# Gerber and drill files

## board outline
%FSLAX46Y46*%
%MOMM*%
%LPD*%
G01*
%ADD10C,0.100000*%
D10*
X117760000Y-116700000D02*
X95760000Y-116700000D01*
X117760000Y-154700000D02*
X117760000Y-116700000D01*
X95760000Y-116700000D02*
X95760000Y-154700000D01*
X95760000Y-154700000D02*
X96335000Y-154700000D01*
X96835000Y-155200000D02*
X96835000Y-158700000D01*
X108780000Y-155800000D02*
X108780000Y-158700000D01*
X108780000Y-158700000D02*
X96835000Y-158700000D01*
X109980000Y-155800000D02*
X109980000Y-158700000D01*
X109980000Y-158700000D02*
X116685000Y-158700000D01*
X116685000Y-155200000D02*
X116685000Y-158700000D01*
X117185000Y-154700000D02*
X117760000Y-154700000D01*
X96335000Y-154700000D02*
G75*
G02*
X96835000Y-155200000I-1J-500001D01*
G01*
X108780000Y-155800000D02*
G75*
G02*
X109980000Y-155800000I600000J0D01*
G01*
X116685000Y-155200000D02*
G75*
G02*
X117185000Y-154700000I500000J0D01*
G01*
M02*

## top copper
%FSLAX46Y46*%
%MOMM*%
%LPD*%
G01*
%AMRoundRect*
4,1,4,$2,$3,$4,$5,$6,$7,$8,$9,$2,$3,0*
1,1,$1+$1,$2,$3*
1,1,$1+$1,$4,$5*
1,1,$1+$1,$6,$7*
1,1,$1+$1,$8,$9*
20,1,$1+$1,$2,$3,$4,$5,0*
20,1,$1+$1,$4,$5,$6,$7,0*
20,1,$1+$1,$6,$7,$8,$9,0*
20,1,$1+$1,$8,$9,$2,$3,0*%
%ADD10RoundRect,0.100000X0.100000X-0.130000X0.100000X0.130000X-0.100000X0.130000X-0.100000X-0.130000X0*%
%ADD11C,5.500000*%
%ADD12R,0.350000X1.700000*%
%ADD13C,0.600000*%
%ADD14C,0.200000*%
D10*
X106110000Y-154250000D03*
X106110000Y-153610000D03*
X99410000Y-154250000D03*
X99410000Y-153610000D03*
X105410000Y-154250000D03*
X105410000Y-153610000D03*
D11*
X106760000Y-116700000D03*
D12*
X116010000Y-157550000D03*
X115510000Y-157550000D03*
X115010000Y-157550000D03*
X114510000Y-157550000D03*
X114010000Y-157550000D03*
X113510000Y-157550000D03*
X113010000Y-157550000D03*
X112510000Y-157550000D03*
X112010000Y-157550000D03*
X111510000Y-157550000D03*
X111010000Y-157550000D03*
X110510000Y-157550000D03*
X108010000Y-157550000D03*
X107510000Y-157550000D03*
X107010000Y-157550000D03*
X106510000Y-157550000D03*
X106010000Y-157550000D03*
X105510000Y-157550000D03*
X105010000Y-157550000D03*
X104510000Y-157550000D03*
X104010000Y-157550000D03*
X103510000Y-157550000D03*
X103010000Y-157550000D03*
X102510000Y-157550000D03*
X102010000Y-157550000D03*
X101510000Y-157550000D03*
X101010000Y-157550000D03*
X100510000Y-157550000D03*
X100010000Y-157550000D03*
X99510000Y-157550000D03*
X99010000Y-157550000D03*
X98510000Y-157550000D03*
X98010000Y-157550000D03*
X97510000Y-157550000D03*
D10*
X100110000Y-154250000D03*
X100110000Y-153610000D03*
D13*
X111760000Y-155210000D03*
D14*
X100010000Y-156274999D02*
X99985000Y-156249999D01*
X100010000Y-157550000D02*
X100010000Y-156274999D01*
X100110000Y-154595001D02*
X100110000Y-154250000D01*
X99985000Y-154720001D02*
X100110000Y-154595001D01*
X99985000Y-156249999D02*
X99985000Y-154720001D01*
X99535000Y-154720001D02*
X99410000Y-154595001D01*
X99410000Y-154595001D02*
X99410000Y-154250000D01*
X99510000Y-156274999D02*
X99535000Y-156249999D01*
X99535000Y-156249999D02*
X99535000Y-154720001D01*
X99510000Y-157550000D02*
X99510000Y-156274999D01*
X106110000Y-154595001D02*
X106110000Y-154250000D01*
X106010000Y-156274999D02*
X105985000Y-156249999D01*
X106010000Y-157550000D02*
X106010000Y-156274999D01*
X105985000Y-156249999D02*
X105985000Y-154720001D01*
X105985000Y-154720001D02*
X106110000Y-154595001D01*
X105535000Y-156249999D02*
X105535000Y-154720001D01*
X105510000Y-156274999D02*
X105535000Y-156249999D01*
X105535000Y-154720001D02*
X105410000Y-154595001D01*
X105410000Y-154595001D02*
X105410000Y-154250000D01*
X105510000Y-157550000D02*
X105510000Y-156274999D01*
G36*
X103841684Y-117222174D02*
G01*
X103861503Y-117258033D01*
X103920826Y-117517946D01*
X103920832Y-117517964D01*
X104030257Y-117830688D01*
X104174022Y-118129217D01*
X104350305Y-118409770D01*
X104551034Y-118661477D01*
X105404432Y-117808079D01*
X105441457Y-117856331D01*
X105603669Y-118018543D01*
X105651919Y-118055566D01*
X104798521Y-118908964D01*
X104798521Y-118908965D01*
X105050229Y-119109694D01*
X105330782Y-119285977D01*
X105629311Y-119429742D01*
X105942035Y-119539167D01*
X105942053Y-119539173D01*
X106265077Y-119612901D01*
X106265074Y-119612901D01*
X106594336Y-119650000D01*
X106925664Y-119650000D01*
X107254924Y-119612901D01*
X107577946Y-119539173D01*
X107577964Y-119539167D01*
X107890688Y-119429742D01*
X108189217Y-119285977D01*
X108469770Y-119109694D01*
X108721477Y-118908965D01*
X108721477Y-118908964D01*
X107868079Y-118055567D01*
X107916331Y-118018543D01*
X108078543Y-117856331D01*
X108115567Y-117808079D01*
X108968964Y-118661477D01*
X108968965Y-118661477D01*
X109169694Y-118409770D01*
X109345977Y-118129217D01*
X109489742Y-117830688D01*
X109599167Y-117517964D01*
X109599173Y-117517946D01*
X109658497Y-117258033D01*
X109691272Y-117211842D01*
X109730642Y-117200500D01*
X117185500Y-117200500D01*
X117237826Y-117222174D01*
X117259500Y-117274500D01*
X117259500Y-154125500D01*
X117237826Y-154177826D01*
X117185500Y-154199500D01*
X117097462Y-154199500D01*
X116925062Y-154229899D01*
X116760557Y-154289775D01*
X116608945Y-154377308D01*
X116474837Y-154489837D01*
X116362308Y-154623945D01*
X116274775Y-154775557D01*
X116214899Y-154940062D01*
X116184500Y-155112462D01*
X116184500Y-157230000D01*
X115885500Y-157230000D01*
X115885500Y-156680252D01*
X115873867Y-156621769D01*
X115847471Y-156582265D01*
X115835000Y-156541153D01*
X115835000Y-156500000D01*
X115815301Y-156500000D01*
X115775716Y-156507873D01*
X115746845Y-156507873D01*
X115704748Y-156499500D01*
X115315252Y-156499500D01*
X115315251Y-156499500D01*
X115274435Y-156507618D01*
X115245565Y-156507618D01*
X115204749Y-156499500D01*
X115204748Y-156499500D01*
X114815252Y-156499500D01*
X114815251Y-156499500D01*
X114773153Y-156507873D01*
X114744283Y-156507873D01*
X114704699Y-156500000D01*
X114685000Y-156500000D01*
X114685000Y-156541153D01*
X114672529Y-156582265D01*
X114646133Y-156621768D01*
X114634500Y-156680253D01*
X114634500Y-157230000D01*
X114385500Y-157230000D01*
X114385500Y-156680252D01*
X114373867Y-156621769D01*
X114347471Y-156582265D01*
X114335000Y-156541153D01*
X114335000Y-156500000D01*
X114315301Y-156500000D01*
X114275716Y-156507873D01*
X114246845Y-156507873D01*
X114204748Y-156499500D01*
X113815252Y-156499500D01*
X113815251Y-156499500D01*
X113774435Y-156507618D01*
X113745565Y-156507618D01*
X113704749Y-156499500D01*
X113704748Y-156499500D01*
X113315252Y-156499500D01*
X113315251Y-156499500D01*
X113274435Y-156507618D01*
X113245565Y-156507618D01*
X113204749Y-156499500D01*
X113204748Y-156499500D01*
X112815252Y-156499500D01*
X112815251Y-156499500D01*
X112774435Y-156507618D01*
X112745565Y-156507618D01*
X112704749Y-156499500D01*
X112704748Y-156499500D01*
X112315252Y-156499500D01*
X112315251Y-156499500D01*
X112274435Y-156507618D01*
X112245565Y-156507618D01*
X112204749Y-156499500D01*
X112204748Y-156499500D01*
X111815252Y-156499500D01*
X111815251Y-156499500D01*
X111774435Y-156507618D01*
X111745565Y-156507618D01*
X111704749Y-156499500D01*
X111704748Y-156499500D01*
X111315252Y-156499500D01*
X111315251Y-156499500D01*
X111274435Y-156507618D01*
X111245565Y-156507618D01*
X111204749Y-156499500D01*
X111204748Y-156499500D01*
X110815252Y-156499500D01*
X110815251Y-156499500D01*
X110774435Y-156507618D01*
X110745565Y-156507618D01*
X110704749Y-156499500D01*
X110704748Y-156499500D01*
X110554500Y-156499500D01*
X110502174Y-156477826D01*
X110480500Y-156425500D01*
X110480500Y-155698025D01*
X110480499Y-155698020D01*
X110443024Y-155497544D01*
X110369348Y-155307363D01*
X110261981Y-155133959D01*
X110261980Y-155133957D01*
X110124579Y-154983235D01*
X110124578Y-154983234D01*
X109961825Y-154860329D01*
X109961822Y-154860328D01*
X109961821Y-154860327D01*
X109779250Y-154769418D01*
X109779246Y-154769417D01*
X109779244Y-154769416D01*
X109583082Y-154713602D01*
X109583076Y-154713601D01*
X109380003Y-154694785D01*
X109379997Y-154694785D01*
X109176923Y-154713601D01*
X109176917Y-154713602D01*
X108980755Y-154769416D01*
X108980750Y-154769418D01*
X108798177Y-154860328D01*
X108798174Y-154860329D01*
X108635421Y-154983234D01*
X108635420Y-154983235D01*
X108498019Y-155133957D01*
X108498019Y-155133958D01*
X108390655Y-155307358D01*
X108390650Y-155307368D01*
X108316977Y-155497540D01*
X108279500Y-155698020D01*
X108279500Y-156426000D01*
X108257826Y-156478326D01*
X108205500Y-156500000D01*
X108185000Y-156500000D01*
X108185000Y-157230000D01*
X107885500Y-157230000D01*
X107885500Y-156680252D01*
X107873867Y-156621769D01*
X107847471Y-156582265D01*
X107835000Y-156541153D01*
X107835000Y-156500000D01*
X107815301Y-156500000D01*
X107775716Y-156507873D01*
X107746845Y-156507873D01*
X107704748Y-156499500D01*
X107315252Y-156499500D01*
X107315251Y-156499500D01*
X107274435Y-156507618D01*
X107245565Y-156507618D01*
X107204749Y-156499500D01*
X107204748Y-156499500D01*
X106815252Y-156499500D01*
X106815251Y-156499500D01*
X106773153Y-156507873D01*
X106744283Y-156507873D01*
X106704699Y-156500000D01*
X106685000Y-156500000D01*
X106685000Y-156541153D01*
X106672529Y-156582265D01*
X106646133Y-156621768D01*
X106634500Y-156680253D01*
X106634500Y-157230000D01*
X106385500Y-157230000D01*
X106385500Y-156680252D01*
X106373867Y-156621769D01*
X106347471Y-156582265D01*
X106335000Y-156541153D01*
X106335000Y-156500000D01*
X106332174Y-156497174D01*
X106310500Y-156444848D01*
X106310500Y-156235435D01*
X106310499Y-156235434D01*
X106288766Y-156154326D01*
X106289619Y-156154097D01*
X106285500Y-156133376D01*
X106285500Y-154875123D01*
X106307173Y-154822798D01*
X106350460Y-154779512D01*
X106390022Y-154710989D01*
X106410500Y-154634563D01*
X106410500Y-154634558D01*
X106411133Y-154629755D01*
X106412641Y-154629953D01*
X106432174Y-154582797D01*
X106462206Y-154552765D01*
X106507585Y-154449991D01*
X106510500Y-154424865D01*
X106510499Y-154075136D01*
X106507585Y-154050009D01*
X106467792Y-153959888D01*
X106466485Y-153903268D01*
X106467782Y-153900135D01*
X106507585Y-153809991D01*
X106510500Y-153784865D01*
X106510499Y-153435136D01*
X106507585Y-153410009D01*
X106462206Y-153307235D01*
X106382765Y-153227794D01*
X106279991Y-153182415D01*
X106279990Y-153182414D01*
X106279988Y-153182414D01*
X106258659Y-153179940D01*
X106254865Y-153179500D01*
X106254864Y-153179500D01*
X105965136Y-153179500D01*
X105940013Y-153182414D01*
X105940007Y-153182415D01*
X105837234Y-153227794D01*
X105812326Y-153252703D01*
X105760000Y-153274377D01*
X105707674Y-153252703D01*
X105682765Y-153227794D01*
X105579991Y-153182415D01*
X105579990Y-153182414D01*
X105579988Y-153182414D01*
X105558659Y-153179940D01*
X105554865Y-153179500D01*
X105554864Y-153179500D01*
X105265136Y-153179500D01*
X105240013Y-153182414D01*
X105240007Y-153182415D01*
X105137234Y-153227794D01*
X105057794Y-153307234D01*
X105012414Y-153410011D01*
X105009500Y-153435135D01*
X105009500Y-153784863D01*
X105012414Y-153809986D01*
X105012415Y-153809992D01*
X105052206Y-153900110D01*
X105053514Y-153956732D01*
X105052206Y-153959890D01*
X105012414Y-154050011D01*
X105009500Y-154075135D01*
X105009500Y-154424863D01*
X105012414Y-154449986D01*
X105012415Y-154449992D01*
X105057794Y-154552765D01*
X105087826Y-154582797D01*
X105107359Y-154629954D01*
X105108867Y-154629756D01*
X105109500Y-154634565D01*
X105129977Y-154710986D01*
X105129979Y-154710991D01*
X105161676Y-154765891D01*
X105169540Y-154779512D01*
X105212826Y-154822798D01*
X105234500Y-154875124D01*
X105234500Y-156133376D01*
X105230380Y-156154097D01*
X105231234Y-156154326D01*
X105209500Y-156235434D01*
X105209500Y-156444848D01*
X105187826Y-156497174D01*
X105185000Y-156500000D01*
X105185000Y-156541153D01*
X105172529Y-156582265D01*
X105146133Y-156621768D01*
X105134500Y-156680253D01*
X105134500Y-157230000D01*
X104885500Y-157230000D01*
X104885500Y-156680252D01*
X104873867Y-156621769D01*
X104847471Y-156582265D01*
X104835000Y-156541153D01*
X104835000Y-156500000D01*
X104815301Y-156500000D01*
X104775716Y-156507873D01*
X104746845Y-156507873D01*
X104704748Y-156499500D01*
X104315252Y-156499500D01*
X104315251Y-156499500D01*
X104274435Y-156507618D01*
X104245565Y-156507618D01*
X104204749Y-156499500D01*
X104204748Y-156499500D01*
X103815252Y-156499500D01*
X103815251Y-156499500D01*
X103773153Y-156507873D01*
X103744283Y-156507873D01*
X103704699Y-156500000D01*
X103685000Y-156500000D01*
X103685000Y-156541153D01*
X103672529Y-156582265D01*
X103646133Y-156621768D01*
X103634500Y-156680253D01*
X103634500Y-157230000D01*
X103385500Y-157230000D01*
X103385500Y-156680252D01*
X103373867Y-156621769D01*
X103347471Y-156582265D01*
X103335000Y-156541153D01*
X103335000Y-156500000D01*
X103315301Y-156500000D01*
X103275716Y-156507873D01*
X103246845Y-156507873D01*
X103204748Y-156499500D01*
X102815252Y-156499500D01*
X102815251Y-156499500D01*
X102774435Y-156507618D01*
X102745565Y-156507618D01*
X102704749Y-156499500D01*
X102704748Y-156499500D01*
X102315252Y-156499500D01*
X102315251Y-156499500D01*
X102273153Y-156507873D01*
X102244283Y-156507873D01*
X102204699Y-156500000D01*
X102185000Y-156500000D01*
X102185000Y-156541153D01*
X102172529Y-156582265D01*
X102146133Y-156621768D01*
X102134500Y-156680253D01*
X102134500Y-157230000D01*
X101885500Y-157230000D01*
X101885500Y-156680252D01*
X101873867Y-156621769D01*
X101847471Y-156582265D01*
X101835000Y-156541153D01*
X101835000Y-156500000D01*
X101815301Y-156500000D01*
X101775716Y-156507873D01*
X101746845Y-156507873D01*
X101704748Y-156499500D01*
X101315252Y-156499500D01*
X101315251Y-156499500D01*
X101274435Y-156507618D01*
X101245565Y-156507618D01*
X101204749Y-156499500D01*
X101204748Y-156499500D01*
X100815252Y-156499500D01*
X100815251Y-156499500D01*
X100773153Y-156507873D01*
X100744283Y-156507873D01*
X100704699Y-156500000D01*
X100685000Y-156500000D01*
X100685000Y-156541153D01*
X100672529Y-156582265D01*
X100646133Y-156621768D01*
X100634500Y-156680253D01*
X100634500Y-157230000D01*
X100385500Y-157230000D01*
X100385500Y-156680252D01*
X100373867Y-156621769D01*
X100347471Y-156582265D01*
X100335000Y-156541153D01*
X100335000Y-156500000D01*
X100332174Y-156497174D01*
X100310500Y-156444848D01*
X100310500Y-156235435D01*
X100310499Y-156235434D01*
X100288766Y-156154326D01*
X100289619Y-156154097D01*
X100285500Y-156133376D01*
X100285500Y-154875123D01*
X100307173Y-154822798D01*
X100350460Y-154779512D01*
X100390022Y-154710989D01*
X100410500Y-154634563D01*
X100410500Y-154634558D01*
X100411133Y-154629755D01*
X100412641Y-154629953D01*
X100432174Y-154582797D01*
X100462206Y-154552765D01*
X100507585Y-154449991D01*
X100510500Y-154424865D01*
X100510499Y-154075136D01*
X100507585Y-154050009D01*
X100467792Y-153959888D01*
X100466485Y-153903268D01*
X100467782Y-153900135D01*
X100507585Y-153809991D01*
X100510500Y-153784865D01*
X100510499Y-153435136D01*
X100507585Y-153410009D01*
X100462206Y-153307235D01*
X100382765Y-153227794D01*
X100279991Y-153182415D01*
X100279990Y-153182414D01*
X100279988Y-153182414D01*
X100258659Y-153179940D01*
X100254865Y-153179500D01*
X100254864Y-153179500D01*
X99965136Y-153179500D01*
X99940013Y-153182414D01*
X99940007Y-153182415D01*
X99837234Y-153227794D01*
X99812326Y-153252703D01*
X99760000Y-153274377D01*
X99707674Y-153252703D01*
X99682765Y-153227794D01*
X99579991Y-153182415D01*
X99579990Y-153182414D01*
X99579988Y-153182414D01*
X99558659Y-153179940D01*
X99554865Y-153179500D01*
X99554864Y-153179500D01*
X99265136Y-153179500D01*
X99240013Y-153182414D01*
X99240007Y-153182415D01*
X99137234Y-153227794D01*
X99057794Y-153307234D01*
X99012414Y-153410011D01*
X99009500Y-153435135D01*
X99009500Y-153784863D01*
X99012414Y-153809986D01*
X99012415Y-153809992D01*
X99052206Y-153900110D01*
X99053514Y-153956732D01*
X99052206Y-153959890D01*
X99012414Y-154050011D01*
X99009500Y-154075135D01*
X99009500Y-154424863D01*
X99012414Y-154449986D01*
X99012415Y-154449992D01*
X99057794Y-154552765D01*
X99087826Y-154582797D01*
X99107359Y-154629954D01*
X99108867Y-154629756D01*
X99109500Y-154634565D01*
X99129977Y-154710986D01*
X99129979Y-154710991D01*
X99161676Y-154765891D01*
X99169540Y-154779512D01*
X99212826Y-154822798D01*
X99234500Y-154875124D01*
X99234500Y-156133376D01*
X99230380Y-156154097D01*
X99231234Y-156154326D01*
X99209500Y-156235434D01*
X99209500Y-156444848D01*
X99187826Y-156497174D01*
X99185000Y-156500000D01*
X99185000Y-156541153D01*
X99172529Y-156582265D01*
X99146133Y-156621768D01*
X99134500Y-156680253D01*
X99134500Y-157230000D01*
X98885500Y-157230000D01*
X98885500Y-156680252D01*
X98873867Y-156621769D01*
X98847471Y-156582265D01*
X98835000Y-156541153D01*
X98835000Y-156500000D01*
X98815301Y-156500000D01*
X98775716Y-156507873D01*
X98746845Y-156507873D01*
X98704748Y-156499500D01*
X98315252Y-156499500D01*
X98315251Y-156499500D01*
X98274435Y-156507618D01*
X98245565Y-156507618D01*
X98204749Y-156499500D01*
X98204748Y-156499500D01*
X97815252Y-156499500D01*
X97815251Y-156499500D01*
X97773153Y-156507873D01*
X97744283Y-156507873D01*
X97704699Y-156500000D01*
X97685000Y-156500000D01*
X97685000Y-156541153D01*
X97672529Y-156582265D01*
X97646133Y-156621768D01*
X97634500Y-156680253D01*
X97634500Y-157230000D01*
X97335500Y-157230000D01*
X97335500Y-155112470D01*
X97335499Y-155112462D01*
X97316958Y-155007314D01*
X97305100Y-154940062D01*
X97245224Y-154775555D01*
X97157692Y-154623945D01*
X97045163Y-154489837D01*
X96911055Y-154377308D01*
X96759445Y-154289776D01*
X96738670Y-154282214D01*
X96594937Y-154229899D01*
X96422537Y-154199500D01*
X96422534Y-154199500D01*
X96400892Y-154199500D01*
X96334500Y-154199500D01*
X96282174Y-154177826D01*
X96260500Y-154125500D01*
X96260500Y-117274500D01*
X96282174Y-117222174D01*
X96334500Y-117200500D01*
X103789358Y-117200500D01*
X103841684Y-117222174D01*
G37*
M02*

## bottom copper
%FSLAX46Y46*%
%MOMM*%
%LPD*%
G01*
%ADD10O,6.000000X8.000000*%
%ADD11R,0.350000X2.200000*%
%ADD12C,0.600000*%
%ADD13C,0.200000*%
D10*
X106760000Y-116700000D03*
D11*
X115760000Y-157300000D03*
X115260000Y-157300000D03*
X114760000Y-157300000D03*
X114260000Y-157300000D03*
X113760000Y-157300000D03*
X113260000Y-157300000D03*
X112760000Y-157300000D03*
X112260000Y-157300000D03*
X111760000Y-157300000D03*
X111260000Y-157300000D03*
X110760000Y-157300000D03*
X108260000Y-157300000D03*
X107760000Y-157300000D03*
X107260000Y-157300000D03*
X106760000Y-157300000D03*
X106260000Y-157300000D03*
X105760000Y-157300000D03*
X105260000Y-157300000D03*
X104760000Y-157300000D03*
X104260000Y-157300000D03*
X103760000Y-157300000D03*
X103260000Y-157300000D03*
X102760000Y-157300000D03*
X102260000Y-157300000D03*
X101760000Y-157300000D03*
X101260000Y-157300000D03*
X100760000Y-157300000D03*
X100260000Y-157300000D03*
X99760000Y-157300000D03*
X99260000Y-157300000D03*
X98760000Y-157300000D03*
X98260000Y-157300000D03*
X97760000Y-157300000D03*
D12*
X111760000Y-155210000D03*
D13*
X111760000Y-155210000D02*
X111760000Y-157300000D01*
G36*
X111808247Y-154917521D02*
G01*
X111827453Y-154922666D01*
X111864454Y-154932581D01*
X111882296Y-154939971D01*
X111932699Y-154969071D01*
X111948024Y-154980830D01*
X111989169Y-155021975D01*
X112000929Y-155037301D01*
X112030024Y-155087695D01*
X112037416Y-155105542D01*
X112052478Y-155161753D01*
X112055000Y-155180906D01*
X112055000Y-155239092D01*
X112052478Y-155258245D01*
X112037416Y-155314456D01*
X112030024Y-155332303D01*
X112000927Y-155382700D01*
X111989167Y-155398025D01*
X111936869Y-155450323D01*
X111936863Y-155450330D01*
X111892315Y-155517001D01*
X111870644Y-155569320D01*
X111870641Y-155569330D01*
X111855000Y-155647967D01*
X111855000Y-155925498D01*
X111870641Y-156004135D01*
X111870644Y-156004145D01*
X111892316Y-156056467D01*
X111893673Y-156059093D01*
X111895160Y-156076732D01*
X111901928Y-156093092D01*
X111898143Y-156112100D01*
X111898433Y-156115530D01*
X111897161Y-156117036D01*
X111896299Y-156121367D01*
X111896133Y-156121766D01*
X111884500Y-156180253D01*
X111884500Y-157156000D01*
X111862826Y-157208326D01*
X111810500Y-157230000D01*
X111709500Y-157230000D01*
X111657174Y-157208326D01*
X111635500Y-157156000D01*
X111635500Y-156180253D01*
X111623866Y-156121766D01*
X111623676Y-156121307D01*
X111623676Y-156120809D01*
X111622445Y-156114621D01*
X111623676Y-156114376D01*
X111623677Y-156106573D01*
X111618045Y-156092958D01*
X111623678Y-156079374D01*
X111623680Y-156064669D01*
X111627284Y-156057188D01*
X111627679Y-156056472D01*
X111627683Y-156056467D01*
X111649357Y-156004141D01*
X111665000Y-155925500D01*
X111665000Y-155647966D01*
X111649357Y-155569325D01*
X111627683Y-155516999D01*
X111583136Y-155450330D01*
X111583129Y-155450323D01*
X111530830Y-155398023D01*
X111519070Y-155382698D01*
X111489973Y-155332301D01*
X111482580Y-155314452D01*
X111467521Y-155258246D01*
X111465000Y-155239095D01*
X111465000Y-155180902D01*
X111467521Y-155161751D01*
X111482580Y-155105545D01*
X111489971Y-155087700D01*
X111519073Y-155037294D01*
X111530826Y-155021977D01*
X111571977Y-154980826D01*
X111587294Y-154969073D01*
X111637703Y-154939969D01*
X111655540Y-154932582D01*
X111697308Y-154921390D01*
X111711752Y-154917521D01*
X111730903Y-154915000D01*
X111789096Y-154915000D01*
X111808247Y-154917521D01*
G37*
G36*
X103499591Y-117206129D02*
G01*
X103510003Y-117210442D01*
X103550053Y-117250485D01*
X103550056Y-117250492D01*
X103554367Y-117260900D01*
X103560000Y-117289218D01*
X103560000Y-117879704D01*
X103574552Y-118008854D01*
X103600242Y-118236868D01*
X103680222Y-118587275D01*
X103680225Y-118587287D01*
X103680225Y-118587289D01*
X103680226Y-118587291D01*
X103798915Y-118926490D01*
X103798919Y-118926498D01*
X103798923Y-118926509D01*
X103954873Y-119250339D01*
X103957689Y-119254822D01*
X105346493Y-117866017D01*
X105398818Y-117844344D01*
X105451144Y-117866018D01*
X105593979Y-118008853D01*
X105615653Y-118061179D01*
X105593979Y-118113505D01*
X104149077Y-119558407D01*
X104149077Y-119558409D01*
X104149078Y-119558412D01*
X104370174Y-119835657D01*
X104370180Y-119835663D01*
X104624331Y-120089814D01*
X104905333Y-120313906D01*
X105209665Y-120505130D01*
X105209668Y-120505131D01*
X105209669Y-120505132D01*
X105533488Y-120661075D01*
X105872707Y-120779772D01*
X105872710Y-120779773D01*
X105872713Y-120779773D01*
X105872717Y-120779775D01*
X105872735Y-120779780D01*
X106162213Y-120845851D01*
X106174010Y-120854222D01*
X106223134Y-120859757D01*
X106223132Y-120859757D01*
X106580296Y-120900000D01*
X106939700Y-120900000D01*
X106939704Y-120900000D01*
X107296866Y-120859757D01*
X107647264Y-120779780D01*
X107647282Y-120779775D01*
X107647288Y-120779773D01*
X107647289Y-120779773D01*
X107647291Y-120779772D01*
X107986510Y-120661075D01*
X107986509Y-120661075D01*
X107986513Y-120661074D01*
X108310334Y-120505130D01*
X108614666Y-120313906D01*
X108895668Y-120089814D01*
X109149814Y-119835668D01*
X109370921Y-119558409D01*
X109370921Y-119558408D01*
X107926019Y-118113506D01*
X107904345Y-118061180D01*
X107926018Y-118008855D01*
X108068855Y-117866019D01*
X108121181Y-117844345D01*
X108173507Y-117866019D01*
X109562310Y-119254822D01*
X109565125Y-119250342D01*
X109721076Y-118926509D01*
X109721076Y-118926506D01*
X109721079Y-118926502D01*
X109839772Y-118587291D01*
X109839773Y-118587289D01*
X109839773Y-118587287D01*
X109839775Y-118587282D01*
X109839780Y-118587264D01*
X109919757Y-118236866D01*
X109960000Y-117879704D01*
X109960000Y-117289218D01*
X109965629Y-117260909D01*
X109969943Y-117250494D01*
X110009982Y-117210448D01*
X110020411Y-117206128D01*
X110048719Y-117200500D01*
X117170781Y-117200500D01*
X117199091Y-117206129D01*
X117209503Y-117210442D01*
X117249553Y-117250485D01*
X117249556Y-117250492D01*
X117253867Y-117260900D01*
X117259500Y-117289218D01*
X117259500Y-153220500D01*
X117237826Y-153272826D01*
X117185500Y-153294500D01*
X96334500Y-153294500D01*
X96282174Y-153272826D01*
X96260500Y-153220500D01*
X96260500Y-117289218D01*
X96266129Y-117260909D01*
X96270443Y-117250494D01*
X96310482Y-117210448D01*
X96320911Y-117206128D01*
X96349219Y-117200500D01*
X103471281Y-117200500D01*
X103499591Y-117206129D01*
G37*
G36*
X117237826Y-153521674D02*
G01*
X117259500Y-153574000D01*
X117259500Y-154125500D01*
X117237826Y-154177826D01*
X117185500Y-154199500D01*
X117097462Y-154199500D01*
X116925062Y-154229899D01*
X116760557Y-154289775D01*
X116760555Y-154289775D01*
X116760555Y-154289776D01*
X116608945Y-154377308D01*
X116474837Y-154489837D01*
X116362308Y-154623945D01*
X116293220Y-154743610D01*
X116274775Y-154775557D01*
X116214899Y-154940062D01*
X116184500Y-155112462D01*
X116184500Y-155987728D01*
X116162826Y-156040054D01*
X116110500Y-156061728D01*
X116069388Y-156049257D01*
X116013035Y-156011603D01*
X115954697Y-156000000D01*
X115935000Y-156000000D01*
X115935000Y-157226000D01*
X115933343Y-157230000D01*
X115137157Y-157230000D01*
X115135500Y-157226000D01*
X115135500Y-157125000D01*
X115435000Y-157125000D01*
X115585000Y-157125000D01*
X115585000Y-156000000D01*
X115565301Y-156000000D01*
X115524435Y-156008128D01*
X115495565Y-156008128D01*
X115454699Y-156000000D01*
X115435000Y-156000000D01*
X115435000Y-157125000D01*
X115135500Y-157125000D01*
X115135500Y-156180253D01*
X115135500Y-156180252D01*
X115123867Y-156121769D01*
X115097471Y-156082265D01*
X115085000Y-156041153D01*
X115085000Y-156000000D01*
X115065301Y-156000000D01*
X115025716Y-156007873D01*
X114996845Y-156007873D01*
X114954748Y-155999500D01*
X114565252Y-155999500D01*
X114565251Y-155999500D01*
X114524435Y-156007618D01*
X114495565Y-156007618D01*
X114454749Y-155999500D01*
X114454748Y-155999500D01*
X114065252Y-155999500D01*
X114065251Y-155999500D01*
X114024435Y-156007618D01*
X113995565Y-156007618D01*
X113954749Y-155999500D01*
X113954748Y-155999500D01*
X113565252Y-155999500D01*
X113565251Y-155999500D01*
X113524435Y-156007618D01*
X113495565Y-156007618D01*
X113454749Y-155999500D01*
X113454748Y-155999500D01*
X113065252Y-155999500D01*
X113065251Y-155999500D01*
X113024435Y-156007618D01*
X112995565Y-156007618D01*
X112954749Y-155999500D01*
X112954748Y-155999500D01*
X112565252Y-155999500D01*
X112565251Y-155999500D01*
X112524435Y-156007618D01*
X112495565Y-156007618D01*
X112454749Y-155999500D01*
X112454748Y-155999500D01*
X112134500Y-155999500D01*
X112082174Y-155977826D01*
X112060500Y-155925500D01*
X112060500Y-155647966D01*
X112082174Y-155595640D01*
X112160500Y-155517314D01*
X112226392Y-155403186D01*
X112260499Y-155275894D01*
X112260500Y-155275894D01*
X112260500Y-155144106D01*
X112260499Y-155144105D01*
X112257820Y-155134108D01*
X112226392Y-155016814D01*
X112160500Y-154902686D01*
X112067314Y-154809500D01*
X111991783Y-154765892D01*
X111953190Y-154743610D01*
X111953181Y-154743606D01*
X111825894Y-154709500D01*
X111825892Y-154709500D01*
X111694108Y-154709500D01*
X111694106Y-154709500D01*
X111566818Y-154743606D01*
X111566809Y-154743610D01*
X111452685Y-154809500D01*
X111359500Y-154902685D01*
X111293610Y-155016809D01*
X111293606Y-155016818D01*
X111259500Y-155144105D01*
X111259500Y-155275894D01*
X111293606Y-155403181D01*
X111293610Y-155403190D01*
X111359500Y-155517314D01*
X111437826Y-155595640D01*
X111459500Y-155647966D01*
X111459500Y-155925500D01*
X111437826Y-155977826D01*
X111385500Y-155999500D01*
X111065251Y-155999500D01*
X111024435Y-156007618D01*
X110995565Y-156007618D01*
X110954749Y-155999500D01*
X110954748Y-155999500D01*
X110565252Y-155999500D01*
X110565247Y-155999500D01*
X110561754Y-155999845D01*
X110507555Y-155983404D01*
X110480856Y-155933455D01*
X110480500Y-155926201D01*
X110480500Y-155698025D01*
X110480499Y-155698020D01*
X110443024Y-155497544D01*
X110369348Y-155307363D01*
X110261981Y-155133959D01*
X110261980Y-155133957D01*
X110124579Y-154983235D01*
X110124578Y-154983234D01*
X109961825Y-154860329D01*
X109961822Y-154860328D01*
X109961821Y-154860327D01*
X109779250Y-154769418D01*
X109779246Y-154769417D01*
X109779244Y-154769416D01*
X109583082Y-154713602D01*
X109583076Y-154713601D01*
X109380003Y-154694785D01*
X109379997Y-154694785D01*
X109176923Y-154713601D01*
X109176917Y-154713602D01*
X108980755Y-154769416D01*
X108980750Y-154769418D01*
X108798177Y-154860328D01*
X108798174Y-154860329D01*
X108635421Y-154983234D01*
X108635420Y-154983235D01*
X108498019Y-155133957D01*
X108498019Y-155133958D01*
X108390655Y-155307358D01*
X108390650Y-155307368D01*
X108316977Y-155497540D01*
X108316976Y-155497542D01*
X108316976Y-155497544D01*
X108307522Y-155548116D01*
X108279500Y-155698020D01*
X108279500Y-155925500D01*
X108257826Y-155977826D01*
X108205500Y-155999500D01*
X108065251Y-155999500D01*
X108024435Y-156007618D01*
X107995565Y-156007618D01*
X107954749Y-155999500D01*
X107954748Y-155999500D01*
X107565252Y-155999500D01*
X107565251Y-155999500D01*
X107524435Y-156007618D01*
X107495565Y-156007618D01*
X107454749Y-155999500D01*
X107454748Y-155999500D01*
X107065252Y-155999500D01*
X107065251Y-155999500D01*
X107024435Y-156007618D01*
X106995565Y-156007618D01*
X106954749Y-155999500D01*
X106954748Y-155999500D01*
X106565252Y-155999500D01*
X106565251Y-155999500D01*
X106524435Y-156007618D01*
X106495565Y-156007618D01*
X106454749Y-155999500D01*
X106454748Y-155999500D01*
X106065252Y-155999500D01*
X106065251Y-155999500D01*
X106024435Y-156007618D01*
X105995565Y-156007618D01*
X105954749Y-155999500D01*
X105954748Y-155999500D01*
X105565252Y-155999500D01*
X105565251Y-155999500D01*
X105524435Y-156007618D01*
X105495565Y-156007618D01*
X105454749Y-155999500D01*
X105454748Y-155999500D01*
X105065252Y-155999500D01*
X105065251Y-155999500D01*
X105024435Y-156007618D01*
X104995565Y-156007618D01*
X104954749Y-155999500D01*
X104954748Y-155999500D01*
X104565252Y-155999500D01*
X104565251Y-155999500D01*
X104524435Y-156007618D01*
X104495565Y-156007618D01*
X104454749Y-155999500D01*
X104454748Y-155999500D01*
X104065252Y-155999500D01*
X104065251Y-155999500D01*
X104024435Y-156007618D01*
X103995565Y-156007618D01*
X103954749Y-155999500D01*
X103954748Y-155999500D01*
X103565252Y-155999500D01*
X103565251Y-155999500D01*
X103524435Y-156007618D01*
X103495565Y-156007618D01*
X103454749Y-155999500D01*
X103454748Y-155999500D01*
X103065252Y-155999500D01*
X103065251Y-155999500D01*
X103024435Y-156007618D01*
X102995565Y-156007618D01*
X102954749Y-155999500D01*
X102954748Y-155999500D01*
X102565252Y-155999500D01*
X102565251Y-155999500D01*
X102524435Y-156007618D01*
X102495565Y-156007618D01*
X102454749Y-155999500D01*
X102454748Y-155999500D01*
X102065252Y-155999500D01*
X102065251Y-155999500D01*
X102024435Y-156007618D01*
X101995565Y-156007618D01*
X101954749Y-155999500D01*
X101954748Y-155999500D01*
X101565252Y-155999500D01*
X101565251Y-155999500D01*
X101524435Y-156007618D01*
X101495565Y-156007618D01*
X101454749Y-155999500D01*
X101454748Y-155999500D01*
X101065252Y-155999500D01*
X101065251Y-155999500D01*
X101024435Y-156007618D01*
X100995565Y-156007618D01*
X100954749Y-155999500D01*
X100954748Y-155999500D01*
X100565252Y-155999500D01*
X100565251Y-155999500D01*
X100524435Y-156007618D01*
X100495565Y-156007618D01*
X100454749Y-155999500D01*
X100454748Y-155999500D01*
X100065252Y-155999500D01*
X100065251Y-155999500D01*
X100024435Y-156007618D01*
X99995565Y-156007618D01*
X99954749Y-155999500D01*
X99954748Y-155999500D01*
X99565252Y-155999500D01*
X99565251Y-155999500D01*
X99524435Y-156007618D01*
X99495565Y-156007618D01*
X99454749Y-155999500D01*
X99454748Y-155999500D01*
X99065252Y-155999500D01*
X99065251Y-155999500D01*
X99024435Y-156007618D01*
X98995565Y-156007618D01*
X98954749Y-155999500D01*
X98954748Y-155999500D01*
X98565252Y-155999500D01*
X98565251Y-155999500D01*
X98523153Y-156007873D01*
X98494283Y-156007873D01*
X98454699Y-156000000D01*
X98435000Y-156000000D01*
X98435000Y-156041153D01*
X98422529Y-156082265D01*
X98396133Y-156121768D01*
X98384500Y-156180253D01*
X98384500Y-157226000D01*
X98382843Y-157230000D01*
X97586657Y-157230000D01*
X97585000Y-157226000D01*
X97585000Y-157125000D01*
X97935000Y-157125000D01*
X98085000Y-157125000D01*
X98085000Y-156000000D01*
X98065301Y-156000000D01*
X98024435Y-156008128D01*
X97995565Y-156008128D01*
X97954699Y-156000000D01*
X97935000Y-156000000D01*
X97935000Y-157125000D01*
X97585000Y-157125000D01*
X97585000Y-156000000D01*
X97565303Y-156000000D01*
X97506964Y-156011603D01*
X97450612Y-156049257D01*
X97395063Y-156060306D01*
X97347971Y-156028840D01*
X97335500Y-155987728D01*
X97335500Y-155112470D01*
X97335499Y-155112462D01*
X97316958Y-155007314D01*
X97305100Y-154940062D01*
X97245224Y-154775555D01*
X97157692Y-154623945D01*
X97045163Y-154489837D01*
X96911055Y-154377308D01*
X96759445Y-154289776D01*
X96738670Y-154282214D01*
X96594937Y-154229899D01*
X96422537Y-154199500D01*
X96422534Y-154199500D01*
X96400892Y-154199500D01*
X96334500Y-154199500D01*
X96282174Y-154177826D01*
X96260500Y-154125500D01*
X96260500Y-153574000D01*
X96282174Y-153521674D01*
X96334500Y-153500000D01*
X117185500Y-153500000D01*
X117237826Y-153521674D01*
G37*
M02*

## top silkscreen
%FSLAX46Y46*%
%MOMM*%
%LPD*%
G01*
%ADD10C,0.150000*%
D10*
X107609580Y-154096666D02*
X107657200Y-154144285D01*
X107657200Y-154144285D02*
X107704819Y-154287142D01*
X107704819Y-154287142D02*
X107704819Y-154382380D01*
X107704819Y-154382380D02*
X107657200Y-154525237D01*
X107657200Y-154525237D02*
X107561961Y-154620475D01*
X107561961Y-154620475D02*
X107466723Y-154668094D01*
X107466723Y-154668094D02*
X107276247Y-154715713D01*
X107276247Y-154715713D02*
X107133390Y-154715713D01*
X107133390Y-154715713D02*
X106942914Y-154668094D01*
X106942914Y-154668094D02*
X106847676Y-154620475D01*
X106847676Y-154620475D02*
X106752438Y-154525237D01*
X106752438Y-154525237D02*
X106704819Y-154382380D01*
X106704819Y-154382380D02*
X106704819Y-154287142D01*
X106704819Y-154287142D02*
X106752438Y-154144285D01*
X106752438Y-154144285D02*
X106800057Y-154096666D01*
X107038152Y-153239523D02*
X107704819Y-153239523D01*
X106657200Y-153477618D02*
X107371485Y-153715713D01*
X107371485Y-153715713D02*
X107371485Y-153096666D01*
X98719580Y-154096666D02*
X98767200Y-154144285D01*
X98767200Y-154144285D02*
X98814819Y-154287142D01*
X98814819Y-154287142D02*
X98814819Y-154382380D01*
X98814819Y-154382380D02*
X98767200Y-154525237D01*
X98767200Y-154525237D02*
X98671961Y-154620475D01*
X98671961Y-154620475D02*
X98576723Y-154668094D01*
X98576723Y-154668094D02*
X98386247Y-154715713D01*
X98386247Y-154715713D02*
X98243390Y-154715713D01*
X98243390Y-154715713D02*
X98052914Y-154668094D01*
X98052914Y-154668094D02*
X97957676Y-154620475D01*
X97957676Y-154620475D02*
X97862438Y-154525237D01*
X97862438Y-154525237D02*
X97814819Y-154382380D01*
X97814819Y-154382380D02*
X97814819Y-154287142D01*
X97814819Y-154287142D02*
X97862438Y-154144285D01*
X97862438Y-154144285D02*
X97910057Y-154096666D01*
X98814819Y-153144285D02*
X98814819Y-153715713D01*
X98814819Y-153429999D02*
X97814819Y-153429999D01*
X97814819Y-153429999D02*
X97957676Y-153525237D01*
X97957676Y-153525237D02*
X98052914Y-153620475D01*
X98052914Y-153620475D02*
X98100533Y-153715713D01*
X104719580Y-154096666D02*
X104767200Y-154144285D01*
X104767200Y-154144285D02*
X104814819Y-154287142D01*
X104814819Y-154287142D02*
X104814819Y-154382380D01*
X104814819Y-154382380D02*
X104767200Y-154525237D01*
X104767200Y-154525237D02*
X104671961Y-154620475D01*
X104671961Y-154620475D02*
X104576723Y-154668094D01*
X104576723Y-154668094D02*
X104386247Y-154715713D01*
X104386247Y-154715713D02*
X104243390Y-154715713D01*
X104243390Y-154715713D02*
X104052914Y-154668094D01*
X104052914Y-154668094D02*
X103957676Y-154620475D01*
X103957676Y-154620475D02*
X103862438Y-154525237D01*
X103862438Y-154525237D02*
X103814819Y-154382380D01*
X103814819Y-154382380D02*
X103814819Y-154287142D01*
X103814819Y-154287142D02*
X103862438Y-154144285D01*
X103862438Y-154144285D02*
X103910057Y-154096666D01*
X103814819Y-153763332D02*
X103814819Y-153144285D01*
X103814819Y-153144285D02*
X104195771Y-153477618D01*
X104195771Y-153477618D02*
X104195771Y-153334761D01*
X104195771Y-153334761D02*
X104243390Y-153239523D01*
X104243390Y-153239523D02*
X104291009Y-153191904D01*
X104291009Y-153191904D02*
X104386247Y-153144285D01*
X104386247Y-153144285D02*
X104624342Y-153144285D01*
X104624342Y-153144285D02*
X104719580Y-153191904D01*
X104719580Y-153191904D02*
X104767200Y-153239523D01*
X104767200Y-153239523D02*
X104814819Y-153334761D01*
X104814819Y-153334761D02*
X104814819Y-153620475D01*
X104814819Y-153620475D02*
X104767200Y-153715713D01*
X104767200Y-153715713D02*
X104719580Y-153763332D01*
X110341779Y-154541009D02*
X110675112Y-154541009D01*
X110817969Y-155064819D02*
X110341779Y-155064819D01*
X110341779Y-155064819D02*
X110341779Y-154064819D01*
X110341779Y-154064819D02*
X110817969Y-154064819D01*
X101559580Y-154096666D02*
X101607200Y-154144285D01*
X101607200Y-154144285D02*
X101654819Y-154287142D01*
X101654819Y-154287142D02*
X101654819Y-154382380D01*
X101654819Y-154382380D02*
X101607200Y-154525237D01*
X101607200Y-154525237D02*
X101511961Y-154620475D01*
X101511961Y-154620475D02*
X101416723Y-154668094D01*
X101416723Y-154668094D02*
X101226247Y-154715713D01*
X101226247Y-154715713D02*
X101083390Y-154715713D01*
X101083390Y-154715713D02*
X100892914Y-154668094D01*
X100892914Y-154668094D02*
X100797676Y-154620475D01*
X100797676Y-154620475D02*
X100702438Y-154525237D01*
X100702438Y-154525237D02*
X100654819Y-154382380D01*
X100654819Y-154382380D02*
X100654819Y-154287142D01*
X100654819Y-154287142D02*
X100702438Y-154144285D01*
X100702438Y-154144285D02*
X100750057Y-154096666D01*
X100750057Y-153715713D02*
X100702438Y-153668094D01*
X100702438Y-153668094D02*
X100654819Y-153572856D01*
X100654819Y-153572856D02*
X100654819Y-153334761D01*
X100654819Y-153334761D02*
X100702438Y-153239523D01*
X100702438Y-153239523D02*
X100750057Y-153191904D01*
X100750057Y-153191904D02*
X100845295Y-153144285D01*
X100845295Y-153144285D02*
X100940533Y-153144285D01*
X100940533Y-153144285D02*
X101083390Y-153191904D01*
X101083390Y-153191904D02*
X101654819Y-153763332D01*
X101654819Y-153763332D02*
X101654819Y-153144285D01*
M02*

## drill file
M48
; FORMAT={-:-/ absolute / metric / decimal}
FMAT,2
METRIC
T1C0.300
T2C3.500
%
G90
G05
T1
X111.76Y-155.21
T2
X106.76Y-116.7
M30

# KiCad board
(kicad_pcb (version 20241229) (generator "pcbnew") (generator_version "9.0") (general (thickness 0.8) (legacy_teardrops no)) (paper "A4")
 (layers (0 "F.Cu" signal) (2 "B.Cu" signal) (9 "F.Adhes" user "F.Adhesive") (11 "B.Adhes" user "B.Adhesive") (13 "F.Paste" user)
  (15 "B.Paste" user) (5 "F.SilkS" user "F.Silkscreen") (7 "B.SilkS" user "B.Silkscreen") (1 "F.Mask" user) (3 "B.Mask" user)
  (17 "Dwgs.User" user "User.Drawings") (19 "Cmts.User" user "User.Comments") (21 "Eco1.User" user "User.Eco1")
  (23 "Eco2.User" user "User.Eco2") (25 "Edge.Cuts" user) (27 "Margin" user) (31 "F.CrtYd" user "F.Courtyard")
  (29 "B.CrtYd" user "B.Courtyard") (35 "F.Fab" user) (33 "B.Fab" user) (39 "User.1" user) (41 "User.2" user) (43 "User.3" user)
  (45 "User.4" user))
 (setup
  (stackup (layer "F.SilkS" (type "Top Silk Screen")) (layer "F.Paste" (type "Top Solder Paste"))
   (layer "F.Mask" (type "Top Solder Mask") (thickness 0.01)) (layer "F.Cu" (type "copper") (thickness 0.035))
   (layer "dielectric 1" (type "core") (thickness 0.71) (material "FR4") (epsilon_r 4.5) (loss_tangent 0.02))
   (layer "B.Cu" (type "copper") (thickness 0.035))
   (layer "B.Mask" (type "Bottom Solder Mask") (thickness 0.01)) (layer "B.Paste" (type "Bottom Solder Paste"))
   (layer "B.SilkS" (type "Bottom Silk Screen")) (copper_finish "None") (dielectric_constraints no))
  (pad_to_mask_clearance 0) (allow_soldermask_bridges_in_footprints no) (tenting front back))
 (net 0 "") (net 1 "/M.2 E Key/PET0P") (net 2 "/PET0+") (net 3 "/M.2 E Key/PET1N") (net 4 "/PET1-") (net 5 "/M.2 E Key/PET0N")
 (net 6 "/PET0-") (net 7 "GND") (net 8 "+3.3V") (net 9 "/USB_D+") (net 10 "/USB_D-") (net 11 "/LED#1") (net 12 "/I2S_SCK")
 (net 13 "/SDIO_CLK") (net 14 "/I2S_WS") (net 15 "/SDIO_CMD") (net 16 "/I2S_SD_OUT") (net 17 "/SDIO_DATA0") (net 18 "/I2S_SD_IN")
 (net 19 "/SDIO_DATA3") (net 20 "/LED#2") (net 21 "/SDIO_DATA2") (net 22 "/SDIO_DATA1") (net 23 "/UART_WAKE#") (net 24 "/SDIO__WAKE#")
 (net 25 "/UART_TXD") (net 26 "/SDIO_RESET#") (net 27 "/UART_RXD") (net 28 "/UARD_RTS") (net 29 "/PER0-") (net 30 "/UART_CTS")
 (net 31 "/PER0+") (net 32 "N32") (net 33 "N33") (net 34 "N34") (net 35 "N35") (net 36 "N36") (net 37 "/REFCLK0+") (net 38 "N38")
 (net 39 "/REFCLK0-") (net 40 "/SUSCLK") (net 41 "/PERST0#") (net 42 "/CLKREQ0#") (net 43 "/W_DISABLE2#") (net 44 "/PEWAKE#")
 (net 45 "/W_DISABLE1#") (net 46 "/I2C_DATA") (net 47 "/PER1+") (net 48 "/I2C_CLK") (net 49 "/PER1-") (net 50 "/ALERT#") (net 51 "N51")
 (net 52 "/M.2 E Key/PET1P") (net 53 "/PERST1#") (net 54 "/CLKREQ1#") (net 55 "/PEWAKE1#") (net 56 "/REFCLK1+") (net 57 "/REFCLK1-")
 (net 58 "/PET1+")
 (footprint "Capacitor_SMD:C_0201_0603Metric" (layer "F.Cu") (at 106.11 153.93 90)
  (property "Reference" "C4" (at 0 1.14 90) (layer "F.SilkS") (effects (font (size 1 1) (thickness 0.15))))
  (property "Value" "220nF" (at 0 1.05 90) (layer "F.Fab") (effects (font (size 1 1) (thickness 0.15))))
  (pad "" smd roundrect (at -0.345 0 90) (size 0.318 0.36) (layers "F.Paste") (roundrect_rratio 0.25))
  (pad "" smd roundrect (at 0.345 0 90) (size 0.318 0.36) (layers "F.Paste") (roundrect_rratio 0.25))
  (pad "1" smd roundrect (at -0.32 0 90) (size 0.46 0.4) (layers "F.Cu" "F.Mask") (roundrect_rratio 0.25) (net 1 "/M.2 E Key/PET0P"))
  (pad "2" smd roundrect (at 0.32 0 90) (size 0.46 0.4) (layers "F.Cu" "F.Mask") (roundrect_rratio 0.25) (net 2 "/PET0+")))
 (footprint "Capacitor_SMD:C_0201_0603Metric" (layer "F.Cu") (at 99.41 153.93 90)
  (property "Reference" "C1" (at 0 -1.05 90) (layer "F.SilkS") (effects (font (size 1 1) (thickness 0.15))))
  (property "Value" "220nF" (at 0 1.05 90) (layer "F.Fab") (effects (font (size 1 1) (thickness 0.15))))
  (pad "" smd roundrect (at -0.345 0 90) (size 0.318 0.36) (layers "F.Paste") (roundrect_rratio 0.25))
  (pad "" smd roundrect (at 0.345 0 90) (size 0.318 0.36) (layers "F.Paste") (roundrect_rratio 0.25))
  (pad "1" smd roundrect (at -0.32 0 90) (size 0.46 0.4) (layers "F.Cu" "F.Mask") (roundrect_rratio 0.25) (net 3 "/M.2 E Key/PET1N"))
  (pad "2" smd roundrect (at 0.32 0 90) (size 0.46 0.4) (layers "F.Cu" "F.Mask") (roundrect_rratio 0.25) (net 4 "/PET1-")))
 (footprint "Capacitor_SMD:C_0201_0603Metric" (layer "F.Cu") (at 105.41 153.93 90)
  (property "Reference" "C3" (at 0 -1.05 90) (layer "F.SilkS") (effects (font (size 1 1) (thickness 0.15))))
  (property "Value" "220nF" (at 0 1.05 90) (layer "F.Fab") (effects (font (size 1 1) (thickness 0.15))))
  (pad "" smd roundrect (at -0.345 0 90) (size 0.318 0.36) (layers "F.Paste") (roundrect_rratio 0.25))
  (pad "" smd roundrect (at 0.345 0 90) (size 0.318 0.36) (layers "F.Paste") (roundrect_rratio 0.25))
  (pad "1" smd roundrect (at -0.32 0 90) (size 0.46 0.4) (layers "F.Cu" "F.Mask") (roundrect_rratio 0.25) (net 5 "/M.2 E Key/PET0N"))
  (pad "2" smd roundrect (at 0.32 0 90) (size 0.46 0.4) (layers "F.Cu" "F.Mask") (roundrect_rratio 0.25) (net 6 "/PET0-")))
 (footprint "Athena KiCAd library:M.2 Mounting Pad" (layer "F.Cu") (at 106.76 116.7)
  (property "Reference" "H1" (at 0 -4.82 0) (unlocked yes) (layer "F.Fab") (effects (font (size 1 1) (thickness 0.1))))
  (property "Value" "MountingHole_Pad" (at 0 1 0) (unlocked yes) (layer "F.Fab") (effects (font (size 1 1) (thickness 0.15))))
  (pad "1" thru_hole circle (at 0 0) (size 5.5 5.5) (drill 3.5) (layers "*.Cu" "*.Mask") (remove_unused_layers no) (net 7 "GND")
   (padstack (mode front_inner_back)
    (layer "Inner" (shape circle) (size 5.5 5.5) (zone_connect -1))
    (layer "B.Cu" (shape oval) (size 6 8) (thermal_bridge_angle 45) (zone_connect -1)))))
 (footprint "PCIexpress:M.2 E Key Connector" (layer "F.Cu") (at 106.76 157.59)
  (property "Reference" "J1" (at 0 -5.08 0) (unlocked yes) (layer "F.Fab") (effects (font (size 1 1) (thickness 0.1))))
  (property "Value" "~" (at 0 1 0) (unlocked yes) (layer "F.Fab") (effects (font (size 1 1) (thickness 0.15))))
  (fp_line (start -11 -2.89) (end -10.425 -2.89) (stroke (width 0.1) (type default)) (layer "Edge.Cuts"))
  (fp_line (start -9.925 -2.39) (end -9.925 1.11) (stroke (width 0.1) (type default)) (layer "Edge.Cuts"))
  (fp_line (start 2.02 -1.79) (end 2.02 1.11) (stroke (width 0.1) (type default)) (layer "Edge.Cuts"))
  (fp_line (start 2.02 1.11) (end -9.925 1.11) (stroke (width 0.1) (type default)) (layer "Edge.Cuts"))
  (fp_line (start 3.22 -1.79) (end 3.22 1.11) (stroke (width 0.1) (type default)) (layer "Edge.Cuts"))
  (fp_line (start 3.22 1.11) (end 9.925 1.11) (stroke (width 0.1) (type default)) (layer "Edge.Cuts"))
  (fp_line (start 9.925 -2.39) (end 9.925 1.11) (stroke (width 0.1) (type default)) (layer "Edge.Cuts"))
  (fp_line (start 10.425 -2.89) (end 11 -2.89) (stroke (width 0.1) (type default)) (layer "Edge.Cuts"))
  (fp_arc (start -10.425 -2.89) (mid -10.071447 -2.743553) (end -9.925 -2.39) (stroke (width 0.1) (type default)) (layer "Edge.Cuts"))
  (fp_arc (start 2.02 -1.79) (mid 2.62 -2.39) (end 3.22 -1.79) (stroke (width 0.1) (type default)) (layer "Edge.Cuts"))
  (fp_arc (start 9.925 -2.39) (mid 10.071447 -2.743553) (end 10.425 -2.89) (stroke (width 0.1) (type default)) (layer "Edge.Cuts"))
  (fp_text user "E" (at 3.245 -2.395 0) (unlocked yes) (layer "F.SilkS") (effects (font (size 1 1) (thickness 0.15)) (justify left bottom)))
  (pad "1" smd rect (at 9.25 -0.04 180) (size 0.35 1.7) (layers "F.Cu") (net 7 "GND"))
  (pad "2" smd rect (at 9 -0.29 180) (size 0.35 2.2) (layers "B.Cu") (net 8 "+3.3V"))
  (pad "3" smd rect (at 8.75 -0.04 180) (size 0.35 1.7) (layers "F.Cu") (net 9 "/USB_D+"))
  (pad "4" smd rect (at 8.5 -0.29 180) (size 0.35 2.2) (layers "B.Cu") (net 8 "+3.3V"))
  (pad "5" smd rect (at 8.25 -0.04 180) (size 0.35 1.7) (layers "F.Cu") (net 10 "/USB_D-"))
  (pad "6" smd rect (at 8 -0.29 180) (size 0.35 2.2) (layers "B.Cu") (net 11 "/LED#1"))
  (pad "7" smd rect (at 7.75 -0.04 180) (size 0.35 1.7) (layers "F.Cu") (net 7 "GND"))
  (pad "8" smd rect (at 7.5 -0.29 180) (size 0.35 2.2) (layers "B.Cu") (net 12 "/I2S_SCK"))
  (pad "9" smd rect (at 7.25 -0.04 180) (size 0.35 1.7) (layers "F.Cu") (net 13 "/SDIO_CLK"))
  (pad "10" smd rect (at 7 -0.29 180) (size 0.35 2.2) (layers "B.Cu") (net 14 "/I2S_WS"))
  (pad "11" smd rect (at 6.75 -0.04 180) (size 0.35 1.7) (layers "F.Cu") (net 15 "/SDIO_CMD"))
  (pad "12" smd rect (at 6.5 -0.29 180) (size 0.35 2.2) (layers "B.Cu") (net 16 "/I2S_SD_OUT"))
  (pad "13" smd rect (at 6.25 -0.04 180) (size 0.35 1.7) (layers "F.Cu") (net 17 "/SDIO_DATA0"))
  (pad "14" smd rect (at 6 -0.29 180) (size 0.35 2.2) (layers "B.Cu") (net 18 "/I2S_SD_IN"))
  (pad "15" smd rect (at 5.75 -0.04 180) (size 0.35 1.7) (layers "F.Cu") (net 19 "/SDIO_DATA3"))
  (pad "16" smd rect (at 5.5 -0.29 180) (size 0.35 2.2) (layers "B.Cu") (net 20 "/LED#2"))
  (pad "17" smd rect (at 5.25 -0.04 180) (size 0.35 1.7) (layers "F.Cu") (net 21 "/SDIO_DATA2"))
  (pad "18" smd rect (at 5 -0.29 180) (size 0.35 2.2) (layers "B.Cu") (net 7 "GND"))
  (pad "19" smd rect (at 4.75 -0.04 180) (size 0.35 1.7) (layers "F.Cu") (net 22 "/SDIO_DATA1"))
  (pad "20" smd rect (at 4.5 -0.29 180) (size 0.35 2.2) (layers "B.Cu") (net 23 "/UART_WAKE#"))
  (pad "21" smd rect (at 4.25 -0.04 180) (size 0.35 1.7) (layers "F.Cu") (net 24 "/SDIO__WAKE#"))
  (pad "22" smd rect (at 4 -0.29 180) (size 0.35 2.2) (layers "B.Cu") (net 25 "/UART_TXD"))
  (pad "23" smd rect (at 3.75 -0.04 180) (size 0.35 1.7) (layers "F.Cu") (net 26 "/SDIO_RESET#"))
  (pad "32" smd rect (at 1.5 -0.29 180) (size 0.35 2.2) (layers "B.Cu") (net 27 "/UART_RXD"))
  (pad "33" smd rect (at 1.25 -0.04 180) (size 0.35 1.7) (layers "F.Cu") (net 7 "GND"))
  (pad "34" smd rect (at 1 -0.29 180) (size 0.35 2.2) (layers "B.Cu") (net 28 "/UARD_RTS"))
  (pad "35" smd rect (at 0.75 -0.04 180) (size 0.35 1.7) (layers "F.Cu") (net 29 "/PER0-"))
  (pad "36" smd rect (at 0.5 -0.29 180) (size 0.35 2.2) (layers "B.Cu") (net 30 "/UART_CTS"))
  (pad "37" smd rect (at 0.25 -0.04 180) (size 0.35 1.7) (layers "F.Cu") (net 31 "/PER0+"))
  (pad "38" smd rect (at 0 -0.29 180) (size 0.35 2.2) (layers "B.Cu") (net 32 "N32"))
  (pad "39" smd rect (at -0.25 -0.04 180) (size 0.35 1.7) (layers "F.Cu") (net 7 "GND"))
  (pad "40" smd rect (at -0.5 -0.29 180) (size 0.35 2.2) (layers "B.Cu") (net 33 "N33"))
  (pad "41" smd rect (at -0.75 -0.04 180) (size 0.35 1.7) (layers "F.Cu") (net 1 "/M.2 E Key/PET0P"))
  (pad "42" smd rect (at -1 -0.29 180) (size 0.35 2.2) (layers "B.Cu") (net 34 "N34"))
  (pad "43" smd rect (at -1.25 -0.04 180) (size 0.35 1.7) (layers "F.Cu") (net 5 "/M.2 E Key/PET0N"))
  (pad "44" smd rect (at -1.5 -0.29 180) (size 0.35 2.2) (layers "B.Cu") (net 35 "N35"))
  (pad "45" smd rect (at -1.75 -0.04 180) (size 0.35 1.7) (layers "F.Cu") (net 7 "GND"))
  (pad "46" smd rect (at -2 -0.29 180) (size 0.35 2.2) (layers "B.Cu") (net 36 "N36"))
  (pad "47" smd rect (at -2.25 -0.04 180) (size 0.35 1.7) (layers "F.Cu") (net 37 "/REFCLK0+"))
  (pad "48" smd rect (at -2.5 -0.29 180) (size 0.35 2.2) (layers "B.Cu") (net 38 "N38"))
  (pad "49" smd rect (at -2.75 -0.04 180) (size 0.35 1.7) (layers "F.Cu") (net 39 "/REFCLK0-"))
  (pad "50" smd rect (at -3 -0.29 180) (size 0.35 2.2) (layers "B.Cu") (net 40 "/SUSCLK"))
  (pad "51" smd rect (at -3.25 -0.04 180) (size 0.35 1.7) (layers "F.Cu") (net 7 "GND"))
  (pad "52" smd rect (at -3.5 -0.29 180) (size 0.35 2.2) (layers "B.Cu") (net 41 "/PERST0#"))
  (pad "53" smd rect (at -3.75 -0.04 180) (size 0.35 1.7) (layers "F.Cu") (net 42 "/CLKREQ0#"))
  (pad "54" smd rect (at -4 -0.29 180) (size 0.35 2.2) (layers "B.Cu") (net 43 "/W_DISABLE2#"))
  (pad "55" smd rect (at -4.25 -0.04 180) (size 0.35 1.7) (layers "F.Cu") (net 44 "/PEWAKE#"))
  (pad "56" smd rect (at -4.5 -0.29 180) (size 0.35 2.2) (layers "B.Cu") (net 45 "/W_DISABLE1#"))
  (pad "57" smd rect (at -4.75 -0.04 180) (size 0.35 1.7) (layers "F.Cu") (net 7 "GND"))
  (pad "58" smd rect (at -5 -0.29 180) (size 0.35 2.2) (layers "B.Cu") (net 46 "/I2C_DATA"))
  (pad "59" smd rect (at -5.25 -0.04 180) (size 0.35 1.7) (layers "F.Cu") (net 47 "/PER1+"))
  (pad "60" smd rect (at -5.5 -0.29 180) (size 0.35 2.2) (layers "B.Cu") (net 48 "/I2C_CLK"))
  (pad "61" smd rect (at -5.75 -0.04 180) (size 0.35 1.7) (layers "F.Cu") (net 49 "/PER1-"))
  (pad "62" smd rect (at -6 -0.29 180) (size 0.35 2.2) (layers "B.Cu") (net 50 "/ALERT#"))
  (pad "63" smd rect (at -6.25 -0.04 180) (size 0.35 1.7) (layers "F.Cu") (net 7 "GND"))
  (pad "64" smd rect (at -6.5 -0.29 180) (size 0.35 2.2) (layers "B.Cu") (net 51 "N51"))
  (pad "65" smd rect (at -6.75 -0.04 180) (size 0.35 1.7) (layers "F.Cu") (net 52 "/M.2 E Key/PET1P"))
  (pad "66" smd rect (at -7 -0.29 180) (size 0.35 2.2) (layers "B.Cu") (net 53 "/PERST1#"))
  (pad "67" smd rect (at -7.25 -0.04 180) (size 0.35 1.7) (layers "F.Cu") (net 3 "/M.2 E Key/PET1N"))
  (pad "68" smd rect (at -7.5 -0.29 180) (size 0.35 2.2) (layers "B.Cu") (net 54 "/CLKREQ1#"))
  (pad "69" smd rect (at -7.75 -0.04 180) (size 0.35 1.7) (layers "F.Cu") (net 7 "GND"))
  (pad "70" smd rect (at -8 -0.29 180) (size 0.35 2.2) (layers "B.Cu") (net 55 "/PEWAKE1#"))
  (pad "71" smd rect (at -8.25 -0.04 180) (size 0.35 1.7) (layers "F.Cu") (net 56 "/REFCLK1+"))
  (pad "72" smd rect (at -8.5 -0.29 180) (size 0.35 2.2) (layers "B.Cu") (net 8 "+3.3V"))
  (pad "73" smd rect (at -8.75 -0.04 180) (size 0.35 1.7) (layers "F.Cu") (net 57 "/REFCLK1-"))
  (pad "74" smd rect (at -9 -0.29 180) (size 0.35 2.2) (layers "B.Cu") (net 8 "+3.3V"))
  (pad "75" smd rect (at -9.25 -0.04 180) (size 0.35 1.7) (layers "F.Cu") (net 7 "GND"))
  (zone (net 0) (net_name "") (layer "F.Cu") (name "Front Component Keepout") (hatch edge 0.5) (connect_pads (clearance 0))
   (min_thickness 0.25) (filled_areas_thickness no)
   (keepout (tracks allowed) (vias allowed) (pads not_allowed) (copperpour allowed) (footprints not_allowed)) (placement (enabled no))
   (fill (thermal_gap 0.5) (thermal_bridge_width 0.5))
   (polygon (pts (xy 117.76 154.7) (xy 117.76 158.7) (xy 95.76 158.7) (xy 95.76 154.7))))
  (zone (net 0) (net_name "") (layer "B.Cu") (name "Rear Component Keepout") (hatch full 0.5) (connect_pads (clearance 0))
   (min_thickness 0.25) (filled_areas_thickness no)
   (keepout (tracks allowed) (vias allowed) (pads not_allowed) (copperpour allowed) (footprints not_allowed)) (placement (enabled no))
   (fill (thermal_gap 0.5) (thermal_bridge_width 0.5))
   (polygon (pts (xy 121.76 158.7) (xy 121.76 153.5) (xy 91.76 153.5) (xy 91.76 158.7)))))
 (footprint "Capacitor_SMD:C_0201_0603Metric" (layer "F.Cu") (at 100.11 153.93 90)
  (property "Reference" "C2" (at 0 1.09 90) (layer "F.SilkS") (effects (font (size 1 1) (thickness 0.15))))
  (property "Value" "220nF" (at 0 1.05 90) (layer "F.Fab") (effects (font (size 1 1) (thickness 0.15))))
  (pad "" smd roundrect (at -0.345 0 90) (size 0.318 0.36) (layers "F.Paste") (roundrect_rratio 0.25))
  (pad "" smd roundrect (at 0.345 0 90) (size 0.318 0.36) (layers "F.Paste") (roundrect_rratio 0.25))
  (pad "1" smd roundrect (at -0.32 0 90) (size 0.46 0.4) (layers "F.Cu" "F.Mask") (roundrect_rratio 0.25) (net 52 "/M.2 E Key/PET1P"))
  (pad "2" smd roundrect (at 0.32 0 90) (size 0.46 0.4) (layers "F.Cu" "F.Mask") (roundrect_rratio 0.25) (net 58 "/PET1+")))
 (gr_line (start 117.76 116.7) (end 95.76 116.7) (stroke (width 0.1) (type default)) (layer "Edge.Cuts"))
 (gr_line (start 117.76 154.7) (end 117.76 116.7) (stroke (width 0.1) (type default)) (layer "Edge.Cuts"))
 (gr_line (start 95.76 116.7) (end 95.76 154.7) (stroke (width 0.1) (type default)) (layer "Edge.Cuts"))
 (segment (start 100.01 156.274999) (end 99.985 156.249999) (width 0.2) (layer "F.Cu") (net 52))
 (segment (start 100.01 157.55) (end 100.01 156.274999) (width 0.2) (layer "F.Cu") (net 52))
 (segment (start 100.11 154.595001) (end 100.11 154.25) (width 0.2) (layer "F.Cu") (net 52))
 (segment (start 99.985 154.720001) (end 100.11 154.595001) (width 0.2) (layer "F.Cu") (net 52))
 (segment (start 99.985 156.249999) (end 99.985 154.720001) (width 0.2) (layer "F.Cu") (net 52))
 (segment (start 99.535 154.720001) (end 99.41 154.595001) (width 0.2) (layer "F.Cu") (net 3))
 (segment (start 99.41 154.595001) (end 99.41 154.25) (width 0.2) (layer "F.Cu") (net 3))
 (segment (start 99.51 156.274999) (end 99.535 156.249999) (width 0.2) (layer "F.Cu") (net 3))
 (segment (start 99.535 156.249999) (end 99.535 154.720001) (width 0.2) (layer "F.Cu") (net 3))
 (segment (start 99.51 157.55) (end 99.51 156.274999) (width 0.2) (layer "F.Cu") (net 3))
 (segment (start 106.11 154.595001) (end 106.11 154.25) (width 0.2) (layer "F.Cu") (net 1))
 (segment (start 106.01 156.274999) (end 105.985 156.249999) (width 0.2) (layer "F.Cu") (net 1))
 (segment (start 106.01 157.55) (end 106.01 156.274999) (width 0.2) (layer "F.Cu") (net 1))
 (segment (start 105.985 156.249999) (end 105.985 154.720001) (width 0.2) (layer "F.Cu") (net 1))
 (segment (start 105.985 154.720001) (end 106.11 154.595001) (width 0.2) (layer "F.Cu") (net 1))
 (segment (start 105.535 156.249999) (end 105.535 154.720001) (width 0.2) (layer "F.Cu") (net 5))
 (segment (start 105.51 156.274999) (end 105.535 156.249999) (width 0.2) (layer "F.Cu") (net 5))
 (segment (start 105.535 154.720001) (end 105.41 154.595001) (width 0.2) (layer "F.Cu") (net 5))
 (segment (start 105.41 154.595001) (end 105.41 154.25) (width 0.2) (layer "F.Cu") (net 5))
 (segment (start 105.51 157.55) (end 105.51 156.274999) (width 0.2) (layer "F.Cu") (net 5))
 (via (at 111.76 155.21) (size 0.6) (drill 0.3) (layers "F.Cu" "B.Cu") (free yes) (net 7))
 (segment (start 111.76 155.21) (end 111.76 157.3) (width 0.2) (layer "B.Cu") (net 7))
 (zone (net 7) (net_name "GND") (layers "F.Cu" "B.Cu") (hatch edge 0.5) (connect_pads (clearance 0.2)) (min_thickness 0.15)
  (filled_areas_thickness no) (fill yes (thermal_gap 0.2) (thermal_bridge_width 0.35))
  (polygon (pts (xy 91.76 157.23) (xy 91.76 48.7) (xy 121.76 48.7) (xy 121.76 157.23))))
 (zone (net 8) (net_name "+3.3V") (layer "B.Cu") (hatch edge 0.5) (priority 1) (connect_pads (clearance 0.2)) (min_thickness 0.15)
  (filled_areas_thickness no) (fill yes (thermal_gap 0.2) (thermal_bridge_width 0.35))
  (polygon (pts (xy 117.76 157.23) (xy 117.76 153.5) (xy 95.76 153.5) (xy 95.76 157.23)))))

